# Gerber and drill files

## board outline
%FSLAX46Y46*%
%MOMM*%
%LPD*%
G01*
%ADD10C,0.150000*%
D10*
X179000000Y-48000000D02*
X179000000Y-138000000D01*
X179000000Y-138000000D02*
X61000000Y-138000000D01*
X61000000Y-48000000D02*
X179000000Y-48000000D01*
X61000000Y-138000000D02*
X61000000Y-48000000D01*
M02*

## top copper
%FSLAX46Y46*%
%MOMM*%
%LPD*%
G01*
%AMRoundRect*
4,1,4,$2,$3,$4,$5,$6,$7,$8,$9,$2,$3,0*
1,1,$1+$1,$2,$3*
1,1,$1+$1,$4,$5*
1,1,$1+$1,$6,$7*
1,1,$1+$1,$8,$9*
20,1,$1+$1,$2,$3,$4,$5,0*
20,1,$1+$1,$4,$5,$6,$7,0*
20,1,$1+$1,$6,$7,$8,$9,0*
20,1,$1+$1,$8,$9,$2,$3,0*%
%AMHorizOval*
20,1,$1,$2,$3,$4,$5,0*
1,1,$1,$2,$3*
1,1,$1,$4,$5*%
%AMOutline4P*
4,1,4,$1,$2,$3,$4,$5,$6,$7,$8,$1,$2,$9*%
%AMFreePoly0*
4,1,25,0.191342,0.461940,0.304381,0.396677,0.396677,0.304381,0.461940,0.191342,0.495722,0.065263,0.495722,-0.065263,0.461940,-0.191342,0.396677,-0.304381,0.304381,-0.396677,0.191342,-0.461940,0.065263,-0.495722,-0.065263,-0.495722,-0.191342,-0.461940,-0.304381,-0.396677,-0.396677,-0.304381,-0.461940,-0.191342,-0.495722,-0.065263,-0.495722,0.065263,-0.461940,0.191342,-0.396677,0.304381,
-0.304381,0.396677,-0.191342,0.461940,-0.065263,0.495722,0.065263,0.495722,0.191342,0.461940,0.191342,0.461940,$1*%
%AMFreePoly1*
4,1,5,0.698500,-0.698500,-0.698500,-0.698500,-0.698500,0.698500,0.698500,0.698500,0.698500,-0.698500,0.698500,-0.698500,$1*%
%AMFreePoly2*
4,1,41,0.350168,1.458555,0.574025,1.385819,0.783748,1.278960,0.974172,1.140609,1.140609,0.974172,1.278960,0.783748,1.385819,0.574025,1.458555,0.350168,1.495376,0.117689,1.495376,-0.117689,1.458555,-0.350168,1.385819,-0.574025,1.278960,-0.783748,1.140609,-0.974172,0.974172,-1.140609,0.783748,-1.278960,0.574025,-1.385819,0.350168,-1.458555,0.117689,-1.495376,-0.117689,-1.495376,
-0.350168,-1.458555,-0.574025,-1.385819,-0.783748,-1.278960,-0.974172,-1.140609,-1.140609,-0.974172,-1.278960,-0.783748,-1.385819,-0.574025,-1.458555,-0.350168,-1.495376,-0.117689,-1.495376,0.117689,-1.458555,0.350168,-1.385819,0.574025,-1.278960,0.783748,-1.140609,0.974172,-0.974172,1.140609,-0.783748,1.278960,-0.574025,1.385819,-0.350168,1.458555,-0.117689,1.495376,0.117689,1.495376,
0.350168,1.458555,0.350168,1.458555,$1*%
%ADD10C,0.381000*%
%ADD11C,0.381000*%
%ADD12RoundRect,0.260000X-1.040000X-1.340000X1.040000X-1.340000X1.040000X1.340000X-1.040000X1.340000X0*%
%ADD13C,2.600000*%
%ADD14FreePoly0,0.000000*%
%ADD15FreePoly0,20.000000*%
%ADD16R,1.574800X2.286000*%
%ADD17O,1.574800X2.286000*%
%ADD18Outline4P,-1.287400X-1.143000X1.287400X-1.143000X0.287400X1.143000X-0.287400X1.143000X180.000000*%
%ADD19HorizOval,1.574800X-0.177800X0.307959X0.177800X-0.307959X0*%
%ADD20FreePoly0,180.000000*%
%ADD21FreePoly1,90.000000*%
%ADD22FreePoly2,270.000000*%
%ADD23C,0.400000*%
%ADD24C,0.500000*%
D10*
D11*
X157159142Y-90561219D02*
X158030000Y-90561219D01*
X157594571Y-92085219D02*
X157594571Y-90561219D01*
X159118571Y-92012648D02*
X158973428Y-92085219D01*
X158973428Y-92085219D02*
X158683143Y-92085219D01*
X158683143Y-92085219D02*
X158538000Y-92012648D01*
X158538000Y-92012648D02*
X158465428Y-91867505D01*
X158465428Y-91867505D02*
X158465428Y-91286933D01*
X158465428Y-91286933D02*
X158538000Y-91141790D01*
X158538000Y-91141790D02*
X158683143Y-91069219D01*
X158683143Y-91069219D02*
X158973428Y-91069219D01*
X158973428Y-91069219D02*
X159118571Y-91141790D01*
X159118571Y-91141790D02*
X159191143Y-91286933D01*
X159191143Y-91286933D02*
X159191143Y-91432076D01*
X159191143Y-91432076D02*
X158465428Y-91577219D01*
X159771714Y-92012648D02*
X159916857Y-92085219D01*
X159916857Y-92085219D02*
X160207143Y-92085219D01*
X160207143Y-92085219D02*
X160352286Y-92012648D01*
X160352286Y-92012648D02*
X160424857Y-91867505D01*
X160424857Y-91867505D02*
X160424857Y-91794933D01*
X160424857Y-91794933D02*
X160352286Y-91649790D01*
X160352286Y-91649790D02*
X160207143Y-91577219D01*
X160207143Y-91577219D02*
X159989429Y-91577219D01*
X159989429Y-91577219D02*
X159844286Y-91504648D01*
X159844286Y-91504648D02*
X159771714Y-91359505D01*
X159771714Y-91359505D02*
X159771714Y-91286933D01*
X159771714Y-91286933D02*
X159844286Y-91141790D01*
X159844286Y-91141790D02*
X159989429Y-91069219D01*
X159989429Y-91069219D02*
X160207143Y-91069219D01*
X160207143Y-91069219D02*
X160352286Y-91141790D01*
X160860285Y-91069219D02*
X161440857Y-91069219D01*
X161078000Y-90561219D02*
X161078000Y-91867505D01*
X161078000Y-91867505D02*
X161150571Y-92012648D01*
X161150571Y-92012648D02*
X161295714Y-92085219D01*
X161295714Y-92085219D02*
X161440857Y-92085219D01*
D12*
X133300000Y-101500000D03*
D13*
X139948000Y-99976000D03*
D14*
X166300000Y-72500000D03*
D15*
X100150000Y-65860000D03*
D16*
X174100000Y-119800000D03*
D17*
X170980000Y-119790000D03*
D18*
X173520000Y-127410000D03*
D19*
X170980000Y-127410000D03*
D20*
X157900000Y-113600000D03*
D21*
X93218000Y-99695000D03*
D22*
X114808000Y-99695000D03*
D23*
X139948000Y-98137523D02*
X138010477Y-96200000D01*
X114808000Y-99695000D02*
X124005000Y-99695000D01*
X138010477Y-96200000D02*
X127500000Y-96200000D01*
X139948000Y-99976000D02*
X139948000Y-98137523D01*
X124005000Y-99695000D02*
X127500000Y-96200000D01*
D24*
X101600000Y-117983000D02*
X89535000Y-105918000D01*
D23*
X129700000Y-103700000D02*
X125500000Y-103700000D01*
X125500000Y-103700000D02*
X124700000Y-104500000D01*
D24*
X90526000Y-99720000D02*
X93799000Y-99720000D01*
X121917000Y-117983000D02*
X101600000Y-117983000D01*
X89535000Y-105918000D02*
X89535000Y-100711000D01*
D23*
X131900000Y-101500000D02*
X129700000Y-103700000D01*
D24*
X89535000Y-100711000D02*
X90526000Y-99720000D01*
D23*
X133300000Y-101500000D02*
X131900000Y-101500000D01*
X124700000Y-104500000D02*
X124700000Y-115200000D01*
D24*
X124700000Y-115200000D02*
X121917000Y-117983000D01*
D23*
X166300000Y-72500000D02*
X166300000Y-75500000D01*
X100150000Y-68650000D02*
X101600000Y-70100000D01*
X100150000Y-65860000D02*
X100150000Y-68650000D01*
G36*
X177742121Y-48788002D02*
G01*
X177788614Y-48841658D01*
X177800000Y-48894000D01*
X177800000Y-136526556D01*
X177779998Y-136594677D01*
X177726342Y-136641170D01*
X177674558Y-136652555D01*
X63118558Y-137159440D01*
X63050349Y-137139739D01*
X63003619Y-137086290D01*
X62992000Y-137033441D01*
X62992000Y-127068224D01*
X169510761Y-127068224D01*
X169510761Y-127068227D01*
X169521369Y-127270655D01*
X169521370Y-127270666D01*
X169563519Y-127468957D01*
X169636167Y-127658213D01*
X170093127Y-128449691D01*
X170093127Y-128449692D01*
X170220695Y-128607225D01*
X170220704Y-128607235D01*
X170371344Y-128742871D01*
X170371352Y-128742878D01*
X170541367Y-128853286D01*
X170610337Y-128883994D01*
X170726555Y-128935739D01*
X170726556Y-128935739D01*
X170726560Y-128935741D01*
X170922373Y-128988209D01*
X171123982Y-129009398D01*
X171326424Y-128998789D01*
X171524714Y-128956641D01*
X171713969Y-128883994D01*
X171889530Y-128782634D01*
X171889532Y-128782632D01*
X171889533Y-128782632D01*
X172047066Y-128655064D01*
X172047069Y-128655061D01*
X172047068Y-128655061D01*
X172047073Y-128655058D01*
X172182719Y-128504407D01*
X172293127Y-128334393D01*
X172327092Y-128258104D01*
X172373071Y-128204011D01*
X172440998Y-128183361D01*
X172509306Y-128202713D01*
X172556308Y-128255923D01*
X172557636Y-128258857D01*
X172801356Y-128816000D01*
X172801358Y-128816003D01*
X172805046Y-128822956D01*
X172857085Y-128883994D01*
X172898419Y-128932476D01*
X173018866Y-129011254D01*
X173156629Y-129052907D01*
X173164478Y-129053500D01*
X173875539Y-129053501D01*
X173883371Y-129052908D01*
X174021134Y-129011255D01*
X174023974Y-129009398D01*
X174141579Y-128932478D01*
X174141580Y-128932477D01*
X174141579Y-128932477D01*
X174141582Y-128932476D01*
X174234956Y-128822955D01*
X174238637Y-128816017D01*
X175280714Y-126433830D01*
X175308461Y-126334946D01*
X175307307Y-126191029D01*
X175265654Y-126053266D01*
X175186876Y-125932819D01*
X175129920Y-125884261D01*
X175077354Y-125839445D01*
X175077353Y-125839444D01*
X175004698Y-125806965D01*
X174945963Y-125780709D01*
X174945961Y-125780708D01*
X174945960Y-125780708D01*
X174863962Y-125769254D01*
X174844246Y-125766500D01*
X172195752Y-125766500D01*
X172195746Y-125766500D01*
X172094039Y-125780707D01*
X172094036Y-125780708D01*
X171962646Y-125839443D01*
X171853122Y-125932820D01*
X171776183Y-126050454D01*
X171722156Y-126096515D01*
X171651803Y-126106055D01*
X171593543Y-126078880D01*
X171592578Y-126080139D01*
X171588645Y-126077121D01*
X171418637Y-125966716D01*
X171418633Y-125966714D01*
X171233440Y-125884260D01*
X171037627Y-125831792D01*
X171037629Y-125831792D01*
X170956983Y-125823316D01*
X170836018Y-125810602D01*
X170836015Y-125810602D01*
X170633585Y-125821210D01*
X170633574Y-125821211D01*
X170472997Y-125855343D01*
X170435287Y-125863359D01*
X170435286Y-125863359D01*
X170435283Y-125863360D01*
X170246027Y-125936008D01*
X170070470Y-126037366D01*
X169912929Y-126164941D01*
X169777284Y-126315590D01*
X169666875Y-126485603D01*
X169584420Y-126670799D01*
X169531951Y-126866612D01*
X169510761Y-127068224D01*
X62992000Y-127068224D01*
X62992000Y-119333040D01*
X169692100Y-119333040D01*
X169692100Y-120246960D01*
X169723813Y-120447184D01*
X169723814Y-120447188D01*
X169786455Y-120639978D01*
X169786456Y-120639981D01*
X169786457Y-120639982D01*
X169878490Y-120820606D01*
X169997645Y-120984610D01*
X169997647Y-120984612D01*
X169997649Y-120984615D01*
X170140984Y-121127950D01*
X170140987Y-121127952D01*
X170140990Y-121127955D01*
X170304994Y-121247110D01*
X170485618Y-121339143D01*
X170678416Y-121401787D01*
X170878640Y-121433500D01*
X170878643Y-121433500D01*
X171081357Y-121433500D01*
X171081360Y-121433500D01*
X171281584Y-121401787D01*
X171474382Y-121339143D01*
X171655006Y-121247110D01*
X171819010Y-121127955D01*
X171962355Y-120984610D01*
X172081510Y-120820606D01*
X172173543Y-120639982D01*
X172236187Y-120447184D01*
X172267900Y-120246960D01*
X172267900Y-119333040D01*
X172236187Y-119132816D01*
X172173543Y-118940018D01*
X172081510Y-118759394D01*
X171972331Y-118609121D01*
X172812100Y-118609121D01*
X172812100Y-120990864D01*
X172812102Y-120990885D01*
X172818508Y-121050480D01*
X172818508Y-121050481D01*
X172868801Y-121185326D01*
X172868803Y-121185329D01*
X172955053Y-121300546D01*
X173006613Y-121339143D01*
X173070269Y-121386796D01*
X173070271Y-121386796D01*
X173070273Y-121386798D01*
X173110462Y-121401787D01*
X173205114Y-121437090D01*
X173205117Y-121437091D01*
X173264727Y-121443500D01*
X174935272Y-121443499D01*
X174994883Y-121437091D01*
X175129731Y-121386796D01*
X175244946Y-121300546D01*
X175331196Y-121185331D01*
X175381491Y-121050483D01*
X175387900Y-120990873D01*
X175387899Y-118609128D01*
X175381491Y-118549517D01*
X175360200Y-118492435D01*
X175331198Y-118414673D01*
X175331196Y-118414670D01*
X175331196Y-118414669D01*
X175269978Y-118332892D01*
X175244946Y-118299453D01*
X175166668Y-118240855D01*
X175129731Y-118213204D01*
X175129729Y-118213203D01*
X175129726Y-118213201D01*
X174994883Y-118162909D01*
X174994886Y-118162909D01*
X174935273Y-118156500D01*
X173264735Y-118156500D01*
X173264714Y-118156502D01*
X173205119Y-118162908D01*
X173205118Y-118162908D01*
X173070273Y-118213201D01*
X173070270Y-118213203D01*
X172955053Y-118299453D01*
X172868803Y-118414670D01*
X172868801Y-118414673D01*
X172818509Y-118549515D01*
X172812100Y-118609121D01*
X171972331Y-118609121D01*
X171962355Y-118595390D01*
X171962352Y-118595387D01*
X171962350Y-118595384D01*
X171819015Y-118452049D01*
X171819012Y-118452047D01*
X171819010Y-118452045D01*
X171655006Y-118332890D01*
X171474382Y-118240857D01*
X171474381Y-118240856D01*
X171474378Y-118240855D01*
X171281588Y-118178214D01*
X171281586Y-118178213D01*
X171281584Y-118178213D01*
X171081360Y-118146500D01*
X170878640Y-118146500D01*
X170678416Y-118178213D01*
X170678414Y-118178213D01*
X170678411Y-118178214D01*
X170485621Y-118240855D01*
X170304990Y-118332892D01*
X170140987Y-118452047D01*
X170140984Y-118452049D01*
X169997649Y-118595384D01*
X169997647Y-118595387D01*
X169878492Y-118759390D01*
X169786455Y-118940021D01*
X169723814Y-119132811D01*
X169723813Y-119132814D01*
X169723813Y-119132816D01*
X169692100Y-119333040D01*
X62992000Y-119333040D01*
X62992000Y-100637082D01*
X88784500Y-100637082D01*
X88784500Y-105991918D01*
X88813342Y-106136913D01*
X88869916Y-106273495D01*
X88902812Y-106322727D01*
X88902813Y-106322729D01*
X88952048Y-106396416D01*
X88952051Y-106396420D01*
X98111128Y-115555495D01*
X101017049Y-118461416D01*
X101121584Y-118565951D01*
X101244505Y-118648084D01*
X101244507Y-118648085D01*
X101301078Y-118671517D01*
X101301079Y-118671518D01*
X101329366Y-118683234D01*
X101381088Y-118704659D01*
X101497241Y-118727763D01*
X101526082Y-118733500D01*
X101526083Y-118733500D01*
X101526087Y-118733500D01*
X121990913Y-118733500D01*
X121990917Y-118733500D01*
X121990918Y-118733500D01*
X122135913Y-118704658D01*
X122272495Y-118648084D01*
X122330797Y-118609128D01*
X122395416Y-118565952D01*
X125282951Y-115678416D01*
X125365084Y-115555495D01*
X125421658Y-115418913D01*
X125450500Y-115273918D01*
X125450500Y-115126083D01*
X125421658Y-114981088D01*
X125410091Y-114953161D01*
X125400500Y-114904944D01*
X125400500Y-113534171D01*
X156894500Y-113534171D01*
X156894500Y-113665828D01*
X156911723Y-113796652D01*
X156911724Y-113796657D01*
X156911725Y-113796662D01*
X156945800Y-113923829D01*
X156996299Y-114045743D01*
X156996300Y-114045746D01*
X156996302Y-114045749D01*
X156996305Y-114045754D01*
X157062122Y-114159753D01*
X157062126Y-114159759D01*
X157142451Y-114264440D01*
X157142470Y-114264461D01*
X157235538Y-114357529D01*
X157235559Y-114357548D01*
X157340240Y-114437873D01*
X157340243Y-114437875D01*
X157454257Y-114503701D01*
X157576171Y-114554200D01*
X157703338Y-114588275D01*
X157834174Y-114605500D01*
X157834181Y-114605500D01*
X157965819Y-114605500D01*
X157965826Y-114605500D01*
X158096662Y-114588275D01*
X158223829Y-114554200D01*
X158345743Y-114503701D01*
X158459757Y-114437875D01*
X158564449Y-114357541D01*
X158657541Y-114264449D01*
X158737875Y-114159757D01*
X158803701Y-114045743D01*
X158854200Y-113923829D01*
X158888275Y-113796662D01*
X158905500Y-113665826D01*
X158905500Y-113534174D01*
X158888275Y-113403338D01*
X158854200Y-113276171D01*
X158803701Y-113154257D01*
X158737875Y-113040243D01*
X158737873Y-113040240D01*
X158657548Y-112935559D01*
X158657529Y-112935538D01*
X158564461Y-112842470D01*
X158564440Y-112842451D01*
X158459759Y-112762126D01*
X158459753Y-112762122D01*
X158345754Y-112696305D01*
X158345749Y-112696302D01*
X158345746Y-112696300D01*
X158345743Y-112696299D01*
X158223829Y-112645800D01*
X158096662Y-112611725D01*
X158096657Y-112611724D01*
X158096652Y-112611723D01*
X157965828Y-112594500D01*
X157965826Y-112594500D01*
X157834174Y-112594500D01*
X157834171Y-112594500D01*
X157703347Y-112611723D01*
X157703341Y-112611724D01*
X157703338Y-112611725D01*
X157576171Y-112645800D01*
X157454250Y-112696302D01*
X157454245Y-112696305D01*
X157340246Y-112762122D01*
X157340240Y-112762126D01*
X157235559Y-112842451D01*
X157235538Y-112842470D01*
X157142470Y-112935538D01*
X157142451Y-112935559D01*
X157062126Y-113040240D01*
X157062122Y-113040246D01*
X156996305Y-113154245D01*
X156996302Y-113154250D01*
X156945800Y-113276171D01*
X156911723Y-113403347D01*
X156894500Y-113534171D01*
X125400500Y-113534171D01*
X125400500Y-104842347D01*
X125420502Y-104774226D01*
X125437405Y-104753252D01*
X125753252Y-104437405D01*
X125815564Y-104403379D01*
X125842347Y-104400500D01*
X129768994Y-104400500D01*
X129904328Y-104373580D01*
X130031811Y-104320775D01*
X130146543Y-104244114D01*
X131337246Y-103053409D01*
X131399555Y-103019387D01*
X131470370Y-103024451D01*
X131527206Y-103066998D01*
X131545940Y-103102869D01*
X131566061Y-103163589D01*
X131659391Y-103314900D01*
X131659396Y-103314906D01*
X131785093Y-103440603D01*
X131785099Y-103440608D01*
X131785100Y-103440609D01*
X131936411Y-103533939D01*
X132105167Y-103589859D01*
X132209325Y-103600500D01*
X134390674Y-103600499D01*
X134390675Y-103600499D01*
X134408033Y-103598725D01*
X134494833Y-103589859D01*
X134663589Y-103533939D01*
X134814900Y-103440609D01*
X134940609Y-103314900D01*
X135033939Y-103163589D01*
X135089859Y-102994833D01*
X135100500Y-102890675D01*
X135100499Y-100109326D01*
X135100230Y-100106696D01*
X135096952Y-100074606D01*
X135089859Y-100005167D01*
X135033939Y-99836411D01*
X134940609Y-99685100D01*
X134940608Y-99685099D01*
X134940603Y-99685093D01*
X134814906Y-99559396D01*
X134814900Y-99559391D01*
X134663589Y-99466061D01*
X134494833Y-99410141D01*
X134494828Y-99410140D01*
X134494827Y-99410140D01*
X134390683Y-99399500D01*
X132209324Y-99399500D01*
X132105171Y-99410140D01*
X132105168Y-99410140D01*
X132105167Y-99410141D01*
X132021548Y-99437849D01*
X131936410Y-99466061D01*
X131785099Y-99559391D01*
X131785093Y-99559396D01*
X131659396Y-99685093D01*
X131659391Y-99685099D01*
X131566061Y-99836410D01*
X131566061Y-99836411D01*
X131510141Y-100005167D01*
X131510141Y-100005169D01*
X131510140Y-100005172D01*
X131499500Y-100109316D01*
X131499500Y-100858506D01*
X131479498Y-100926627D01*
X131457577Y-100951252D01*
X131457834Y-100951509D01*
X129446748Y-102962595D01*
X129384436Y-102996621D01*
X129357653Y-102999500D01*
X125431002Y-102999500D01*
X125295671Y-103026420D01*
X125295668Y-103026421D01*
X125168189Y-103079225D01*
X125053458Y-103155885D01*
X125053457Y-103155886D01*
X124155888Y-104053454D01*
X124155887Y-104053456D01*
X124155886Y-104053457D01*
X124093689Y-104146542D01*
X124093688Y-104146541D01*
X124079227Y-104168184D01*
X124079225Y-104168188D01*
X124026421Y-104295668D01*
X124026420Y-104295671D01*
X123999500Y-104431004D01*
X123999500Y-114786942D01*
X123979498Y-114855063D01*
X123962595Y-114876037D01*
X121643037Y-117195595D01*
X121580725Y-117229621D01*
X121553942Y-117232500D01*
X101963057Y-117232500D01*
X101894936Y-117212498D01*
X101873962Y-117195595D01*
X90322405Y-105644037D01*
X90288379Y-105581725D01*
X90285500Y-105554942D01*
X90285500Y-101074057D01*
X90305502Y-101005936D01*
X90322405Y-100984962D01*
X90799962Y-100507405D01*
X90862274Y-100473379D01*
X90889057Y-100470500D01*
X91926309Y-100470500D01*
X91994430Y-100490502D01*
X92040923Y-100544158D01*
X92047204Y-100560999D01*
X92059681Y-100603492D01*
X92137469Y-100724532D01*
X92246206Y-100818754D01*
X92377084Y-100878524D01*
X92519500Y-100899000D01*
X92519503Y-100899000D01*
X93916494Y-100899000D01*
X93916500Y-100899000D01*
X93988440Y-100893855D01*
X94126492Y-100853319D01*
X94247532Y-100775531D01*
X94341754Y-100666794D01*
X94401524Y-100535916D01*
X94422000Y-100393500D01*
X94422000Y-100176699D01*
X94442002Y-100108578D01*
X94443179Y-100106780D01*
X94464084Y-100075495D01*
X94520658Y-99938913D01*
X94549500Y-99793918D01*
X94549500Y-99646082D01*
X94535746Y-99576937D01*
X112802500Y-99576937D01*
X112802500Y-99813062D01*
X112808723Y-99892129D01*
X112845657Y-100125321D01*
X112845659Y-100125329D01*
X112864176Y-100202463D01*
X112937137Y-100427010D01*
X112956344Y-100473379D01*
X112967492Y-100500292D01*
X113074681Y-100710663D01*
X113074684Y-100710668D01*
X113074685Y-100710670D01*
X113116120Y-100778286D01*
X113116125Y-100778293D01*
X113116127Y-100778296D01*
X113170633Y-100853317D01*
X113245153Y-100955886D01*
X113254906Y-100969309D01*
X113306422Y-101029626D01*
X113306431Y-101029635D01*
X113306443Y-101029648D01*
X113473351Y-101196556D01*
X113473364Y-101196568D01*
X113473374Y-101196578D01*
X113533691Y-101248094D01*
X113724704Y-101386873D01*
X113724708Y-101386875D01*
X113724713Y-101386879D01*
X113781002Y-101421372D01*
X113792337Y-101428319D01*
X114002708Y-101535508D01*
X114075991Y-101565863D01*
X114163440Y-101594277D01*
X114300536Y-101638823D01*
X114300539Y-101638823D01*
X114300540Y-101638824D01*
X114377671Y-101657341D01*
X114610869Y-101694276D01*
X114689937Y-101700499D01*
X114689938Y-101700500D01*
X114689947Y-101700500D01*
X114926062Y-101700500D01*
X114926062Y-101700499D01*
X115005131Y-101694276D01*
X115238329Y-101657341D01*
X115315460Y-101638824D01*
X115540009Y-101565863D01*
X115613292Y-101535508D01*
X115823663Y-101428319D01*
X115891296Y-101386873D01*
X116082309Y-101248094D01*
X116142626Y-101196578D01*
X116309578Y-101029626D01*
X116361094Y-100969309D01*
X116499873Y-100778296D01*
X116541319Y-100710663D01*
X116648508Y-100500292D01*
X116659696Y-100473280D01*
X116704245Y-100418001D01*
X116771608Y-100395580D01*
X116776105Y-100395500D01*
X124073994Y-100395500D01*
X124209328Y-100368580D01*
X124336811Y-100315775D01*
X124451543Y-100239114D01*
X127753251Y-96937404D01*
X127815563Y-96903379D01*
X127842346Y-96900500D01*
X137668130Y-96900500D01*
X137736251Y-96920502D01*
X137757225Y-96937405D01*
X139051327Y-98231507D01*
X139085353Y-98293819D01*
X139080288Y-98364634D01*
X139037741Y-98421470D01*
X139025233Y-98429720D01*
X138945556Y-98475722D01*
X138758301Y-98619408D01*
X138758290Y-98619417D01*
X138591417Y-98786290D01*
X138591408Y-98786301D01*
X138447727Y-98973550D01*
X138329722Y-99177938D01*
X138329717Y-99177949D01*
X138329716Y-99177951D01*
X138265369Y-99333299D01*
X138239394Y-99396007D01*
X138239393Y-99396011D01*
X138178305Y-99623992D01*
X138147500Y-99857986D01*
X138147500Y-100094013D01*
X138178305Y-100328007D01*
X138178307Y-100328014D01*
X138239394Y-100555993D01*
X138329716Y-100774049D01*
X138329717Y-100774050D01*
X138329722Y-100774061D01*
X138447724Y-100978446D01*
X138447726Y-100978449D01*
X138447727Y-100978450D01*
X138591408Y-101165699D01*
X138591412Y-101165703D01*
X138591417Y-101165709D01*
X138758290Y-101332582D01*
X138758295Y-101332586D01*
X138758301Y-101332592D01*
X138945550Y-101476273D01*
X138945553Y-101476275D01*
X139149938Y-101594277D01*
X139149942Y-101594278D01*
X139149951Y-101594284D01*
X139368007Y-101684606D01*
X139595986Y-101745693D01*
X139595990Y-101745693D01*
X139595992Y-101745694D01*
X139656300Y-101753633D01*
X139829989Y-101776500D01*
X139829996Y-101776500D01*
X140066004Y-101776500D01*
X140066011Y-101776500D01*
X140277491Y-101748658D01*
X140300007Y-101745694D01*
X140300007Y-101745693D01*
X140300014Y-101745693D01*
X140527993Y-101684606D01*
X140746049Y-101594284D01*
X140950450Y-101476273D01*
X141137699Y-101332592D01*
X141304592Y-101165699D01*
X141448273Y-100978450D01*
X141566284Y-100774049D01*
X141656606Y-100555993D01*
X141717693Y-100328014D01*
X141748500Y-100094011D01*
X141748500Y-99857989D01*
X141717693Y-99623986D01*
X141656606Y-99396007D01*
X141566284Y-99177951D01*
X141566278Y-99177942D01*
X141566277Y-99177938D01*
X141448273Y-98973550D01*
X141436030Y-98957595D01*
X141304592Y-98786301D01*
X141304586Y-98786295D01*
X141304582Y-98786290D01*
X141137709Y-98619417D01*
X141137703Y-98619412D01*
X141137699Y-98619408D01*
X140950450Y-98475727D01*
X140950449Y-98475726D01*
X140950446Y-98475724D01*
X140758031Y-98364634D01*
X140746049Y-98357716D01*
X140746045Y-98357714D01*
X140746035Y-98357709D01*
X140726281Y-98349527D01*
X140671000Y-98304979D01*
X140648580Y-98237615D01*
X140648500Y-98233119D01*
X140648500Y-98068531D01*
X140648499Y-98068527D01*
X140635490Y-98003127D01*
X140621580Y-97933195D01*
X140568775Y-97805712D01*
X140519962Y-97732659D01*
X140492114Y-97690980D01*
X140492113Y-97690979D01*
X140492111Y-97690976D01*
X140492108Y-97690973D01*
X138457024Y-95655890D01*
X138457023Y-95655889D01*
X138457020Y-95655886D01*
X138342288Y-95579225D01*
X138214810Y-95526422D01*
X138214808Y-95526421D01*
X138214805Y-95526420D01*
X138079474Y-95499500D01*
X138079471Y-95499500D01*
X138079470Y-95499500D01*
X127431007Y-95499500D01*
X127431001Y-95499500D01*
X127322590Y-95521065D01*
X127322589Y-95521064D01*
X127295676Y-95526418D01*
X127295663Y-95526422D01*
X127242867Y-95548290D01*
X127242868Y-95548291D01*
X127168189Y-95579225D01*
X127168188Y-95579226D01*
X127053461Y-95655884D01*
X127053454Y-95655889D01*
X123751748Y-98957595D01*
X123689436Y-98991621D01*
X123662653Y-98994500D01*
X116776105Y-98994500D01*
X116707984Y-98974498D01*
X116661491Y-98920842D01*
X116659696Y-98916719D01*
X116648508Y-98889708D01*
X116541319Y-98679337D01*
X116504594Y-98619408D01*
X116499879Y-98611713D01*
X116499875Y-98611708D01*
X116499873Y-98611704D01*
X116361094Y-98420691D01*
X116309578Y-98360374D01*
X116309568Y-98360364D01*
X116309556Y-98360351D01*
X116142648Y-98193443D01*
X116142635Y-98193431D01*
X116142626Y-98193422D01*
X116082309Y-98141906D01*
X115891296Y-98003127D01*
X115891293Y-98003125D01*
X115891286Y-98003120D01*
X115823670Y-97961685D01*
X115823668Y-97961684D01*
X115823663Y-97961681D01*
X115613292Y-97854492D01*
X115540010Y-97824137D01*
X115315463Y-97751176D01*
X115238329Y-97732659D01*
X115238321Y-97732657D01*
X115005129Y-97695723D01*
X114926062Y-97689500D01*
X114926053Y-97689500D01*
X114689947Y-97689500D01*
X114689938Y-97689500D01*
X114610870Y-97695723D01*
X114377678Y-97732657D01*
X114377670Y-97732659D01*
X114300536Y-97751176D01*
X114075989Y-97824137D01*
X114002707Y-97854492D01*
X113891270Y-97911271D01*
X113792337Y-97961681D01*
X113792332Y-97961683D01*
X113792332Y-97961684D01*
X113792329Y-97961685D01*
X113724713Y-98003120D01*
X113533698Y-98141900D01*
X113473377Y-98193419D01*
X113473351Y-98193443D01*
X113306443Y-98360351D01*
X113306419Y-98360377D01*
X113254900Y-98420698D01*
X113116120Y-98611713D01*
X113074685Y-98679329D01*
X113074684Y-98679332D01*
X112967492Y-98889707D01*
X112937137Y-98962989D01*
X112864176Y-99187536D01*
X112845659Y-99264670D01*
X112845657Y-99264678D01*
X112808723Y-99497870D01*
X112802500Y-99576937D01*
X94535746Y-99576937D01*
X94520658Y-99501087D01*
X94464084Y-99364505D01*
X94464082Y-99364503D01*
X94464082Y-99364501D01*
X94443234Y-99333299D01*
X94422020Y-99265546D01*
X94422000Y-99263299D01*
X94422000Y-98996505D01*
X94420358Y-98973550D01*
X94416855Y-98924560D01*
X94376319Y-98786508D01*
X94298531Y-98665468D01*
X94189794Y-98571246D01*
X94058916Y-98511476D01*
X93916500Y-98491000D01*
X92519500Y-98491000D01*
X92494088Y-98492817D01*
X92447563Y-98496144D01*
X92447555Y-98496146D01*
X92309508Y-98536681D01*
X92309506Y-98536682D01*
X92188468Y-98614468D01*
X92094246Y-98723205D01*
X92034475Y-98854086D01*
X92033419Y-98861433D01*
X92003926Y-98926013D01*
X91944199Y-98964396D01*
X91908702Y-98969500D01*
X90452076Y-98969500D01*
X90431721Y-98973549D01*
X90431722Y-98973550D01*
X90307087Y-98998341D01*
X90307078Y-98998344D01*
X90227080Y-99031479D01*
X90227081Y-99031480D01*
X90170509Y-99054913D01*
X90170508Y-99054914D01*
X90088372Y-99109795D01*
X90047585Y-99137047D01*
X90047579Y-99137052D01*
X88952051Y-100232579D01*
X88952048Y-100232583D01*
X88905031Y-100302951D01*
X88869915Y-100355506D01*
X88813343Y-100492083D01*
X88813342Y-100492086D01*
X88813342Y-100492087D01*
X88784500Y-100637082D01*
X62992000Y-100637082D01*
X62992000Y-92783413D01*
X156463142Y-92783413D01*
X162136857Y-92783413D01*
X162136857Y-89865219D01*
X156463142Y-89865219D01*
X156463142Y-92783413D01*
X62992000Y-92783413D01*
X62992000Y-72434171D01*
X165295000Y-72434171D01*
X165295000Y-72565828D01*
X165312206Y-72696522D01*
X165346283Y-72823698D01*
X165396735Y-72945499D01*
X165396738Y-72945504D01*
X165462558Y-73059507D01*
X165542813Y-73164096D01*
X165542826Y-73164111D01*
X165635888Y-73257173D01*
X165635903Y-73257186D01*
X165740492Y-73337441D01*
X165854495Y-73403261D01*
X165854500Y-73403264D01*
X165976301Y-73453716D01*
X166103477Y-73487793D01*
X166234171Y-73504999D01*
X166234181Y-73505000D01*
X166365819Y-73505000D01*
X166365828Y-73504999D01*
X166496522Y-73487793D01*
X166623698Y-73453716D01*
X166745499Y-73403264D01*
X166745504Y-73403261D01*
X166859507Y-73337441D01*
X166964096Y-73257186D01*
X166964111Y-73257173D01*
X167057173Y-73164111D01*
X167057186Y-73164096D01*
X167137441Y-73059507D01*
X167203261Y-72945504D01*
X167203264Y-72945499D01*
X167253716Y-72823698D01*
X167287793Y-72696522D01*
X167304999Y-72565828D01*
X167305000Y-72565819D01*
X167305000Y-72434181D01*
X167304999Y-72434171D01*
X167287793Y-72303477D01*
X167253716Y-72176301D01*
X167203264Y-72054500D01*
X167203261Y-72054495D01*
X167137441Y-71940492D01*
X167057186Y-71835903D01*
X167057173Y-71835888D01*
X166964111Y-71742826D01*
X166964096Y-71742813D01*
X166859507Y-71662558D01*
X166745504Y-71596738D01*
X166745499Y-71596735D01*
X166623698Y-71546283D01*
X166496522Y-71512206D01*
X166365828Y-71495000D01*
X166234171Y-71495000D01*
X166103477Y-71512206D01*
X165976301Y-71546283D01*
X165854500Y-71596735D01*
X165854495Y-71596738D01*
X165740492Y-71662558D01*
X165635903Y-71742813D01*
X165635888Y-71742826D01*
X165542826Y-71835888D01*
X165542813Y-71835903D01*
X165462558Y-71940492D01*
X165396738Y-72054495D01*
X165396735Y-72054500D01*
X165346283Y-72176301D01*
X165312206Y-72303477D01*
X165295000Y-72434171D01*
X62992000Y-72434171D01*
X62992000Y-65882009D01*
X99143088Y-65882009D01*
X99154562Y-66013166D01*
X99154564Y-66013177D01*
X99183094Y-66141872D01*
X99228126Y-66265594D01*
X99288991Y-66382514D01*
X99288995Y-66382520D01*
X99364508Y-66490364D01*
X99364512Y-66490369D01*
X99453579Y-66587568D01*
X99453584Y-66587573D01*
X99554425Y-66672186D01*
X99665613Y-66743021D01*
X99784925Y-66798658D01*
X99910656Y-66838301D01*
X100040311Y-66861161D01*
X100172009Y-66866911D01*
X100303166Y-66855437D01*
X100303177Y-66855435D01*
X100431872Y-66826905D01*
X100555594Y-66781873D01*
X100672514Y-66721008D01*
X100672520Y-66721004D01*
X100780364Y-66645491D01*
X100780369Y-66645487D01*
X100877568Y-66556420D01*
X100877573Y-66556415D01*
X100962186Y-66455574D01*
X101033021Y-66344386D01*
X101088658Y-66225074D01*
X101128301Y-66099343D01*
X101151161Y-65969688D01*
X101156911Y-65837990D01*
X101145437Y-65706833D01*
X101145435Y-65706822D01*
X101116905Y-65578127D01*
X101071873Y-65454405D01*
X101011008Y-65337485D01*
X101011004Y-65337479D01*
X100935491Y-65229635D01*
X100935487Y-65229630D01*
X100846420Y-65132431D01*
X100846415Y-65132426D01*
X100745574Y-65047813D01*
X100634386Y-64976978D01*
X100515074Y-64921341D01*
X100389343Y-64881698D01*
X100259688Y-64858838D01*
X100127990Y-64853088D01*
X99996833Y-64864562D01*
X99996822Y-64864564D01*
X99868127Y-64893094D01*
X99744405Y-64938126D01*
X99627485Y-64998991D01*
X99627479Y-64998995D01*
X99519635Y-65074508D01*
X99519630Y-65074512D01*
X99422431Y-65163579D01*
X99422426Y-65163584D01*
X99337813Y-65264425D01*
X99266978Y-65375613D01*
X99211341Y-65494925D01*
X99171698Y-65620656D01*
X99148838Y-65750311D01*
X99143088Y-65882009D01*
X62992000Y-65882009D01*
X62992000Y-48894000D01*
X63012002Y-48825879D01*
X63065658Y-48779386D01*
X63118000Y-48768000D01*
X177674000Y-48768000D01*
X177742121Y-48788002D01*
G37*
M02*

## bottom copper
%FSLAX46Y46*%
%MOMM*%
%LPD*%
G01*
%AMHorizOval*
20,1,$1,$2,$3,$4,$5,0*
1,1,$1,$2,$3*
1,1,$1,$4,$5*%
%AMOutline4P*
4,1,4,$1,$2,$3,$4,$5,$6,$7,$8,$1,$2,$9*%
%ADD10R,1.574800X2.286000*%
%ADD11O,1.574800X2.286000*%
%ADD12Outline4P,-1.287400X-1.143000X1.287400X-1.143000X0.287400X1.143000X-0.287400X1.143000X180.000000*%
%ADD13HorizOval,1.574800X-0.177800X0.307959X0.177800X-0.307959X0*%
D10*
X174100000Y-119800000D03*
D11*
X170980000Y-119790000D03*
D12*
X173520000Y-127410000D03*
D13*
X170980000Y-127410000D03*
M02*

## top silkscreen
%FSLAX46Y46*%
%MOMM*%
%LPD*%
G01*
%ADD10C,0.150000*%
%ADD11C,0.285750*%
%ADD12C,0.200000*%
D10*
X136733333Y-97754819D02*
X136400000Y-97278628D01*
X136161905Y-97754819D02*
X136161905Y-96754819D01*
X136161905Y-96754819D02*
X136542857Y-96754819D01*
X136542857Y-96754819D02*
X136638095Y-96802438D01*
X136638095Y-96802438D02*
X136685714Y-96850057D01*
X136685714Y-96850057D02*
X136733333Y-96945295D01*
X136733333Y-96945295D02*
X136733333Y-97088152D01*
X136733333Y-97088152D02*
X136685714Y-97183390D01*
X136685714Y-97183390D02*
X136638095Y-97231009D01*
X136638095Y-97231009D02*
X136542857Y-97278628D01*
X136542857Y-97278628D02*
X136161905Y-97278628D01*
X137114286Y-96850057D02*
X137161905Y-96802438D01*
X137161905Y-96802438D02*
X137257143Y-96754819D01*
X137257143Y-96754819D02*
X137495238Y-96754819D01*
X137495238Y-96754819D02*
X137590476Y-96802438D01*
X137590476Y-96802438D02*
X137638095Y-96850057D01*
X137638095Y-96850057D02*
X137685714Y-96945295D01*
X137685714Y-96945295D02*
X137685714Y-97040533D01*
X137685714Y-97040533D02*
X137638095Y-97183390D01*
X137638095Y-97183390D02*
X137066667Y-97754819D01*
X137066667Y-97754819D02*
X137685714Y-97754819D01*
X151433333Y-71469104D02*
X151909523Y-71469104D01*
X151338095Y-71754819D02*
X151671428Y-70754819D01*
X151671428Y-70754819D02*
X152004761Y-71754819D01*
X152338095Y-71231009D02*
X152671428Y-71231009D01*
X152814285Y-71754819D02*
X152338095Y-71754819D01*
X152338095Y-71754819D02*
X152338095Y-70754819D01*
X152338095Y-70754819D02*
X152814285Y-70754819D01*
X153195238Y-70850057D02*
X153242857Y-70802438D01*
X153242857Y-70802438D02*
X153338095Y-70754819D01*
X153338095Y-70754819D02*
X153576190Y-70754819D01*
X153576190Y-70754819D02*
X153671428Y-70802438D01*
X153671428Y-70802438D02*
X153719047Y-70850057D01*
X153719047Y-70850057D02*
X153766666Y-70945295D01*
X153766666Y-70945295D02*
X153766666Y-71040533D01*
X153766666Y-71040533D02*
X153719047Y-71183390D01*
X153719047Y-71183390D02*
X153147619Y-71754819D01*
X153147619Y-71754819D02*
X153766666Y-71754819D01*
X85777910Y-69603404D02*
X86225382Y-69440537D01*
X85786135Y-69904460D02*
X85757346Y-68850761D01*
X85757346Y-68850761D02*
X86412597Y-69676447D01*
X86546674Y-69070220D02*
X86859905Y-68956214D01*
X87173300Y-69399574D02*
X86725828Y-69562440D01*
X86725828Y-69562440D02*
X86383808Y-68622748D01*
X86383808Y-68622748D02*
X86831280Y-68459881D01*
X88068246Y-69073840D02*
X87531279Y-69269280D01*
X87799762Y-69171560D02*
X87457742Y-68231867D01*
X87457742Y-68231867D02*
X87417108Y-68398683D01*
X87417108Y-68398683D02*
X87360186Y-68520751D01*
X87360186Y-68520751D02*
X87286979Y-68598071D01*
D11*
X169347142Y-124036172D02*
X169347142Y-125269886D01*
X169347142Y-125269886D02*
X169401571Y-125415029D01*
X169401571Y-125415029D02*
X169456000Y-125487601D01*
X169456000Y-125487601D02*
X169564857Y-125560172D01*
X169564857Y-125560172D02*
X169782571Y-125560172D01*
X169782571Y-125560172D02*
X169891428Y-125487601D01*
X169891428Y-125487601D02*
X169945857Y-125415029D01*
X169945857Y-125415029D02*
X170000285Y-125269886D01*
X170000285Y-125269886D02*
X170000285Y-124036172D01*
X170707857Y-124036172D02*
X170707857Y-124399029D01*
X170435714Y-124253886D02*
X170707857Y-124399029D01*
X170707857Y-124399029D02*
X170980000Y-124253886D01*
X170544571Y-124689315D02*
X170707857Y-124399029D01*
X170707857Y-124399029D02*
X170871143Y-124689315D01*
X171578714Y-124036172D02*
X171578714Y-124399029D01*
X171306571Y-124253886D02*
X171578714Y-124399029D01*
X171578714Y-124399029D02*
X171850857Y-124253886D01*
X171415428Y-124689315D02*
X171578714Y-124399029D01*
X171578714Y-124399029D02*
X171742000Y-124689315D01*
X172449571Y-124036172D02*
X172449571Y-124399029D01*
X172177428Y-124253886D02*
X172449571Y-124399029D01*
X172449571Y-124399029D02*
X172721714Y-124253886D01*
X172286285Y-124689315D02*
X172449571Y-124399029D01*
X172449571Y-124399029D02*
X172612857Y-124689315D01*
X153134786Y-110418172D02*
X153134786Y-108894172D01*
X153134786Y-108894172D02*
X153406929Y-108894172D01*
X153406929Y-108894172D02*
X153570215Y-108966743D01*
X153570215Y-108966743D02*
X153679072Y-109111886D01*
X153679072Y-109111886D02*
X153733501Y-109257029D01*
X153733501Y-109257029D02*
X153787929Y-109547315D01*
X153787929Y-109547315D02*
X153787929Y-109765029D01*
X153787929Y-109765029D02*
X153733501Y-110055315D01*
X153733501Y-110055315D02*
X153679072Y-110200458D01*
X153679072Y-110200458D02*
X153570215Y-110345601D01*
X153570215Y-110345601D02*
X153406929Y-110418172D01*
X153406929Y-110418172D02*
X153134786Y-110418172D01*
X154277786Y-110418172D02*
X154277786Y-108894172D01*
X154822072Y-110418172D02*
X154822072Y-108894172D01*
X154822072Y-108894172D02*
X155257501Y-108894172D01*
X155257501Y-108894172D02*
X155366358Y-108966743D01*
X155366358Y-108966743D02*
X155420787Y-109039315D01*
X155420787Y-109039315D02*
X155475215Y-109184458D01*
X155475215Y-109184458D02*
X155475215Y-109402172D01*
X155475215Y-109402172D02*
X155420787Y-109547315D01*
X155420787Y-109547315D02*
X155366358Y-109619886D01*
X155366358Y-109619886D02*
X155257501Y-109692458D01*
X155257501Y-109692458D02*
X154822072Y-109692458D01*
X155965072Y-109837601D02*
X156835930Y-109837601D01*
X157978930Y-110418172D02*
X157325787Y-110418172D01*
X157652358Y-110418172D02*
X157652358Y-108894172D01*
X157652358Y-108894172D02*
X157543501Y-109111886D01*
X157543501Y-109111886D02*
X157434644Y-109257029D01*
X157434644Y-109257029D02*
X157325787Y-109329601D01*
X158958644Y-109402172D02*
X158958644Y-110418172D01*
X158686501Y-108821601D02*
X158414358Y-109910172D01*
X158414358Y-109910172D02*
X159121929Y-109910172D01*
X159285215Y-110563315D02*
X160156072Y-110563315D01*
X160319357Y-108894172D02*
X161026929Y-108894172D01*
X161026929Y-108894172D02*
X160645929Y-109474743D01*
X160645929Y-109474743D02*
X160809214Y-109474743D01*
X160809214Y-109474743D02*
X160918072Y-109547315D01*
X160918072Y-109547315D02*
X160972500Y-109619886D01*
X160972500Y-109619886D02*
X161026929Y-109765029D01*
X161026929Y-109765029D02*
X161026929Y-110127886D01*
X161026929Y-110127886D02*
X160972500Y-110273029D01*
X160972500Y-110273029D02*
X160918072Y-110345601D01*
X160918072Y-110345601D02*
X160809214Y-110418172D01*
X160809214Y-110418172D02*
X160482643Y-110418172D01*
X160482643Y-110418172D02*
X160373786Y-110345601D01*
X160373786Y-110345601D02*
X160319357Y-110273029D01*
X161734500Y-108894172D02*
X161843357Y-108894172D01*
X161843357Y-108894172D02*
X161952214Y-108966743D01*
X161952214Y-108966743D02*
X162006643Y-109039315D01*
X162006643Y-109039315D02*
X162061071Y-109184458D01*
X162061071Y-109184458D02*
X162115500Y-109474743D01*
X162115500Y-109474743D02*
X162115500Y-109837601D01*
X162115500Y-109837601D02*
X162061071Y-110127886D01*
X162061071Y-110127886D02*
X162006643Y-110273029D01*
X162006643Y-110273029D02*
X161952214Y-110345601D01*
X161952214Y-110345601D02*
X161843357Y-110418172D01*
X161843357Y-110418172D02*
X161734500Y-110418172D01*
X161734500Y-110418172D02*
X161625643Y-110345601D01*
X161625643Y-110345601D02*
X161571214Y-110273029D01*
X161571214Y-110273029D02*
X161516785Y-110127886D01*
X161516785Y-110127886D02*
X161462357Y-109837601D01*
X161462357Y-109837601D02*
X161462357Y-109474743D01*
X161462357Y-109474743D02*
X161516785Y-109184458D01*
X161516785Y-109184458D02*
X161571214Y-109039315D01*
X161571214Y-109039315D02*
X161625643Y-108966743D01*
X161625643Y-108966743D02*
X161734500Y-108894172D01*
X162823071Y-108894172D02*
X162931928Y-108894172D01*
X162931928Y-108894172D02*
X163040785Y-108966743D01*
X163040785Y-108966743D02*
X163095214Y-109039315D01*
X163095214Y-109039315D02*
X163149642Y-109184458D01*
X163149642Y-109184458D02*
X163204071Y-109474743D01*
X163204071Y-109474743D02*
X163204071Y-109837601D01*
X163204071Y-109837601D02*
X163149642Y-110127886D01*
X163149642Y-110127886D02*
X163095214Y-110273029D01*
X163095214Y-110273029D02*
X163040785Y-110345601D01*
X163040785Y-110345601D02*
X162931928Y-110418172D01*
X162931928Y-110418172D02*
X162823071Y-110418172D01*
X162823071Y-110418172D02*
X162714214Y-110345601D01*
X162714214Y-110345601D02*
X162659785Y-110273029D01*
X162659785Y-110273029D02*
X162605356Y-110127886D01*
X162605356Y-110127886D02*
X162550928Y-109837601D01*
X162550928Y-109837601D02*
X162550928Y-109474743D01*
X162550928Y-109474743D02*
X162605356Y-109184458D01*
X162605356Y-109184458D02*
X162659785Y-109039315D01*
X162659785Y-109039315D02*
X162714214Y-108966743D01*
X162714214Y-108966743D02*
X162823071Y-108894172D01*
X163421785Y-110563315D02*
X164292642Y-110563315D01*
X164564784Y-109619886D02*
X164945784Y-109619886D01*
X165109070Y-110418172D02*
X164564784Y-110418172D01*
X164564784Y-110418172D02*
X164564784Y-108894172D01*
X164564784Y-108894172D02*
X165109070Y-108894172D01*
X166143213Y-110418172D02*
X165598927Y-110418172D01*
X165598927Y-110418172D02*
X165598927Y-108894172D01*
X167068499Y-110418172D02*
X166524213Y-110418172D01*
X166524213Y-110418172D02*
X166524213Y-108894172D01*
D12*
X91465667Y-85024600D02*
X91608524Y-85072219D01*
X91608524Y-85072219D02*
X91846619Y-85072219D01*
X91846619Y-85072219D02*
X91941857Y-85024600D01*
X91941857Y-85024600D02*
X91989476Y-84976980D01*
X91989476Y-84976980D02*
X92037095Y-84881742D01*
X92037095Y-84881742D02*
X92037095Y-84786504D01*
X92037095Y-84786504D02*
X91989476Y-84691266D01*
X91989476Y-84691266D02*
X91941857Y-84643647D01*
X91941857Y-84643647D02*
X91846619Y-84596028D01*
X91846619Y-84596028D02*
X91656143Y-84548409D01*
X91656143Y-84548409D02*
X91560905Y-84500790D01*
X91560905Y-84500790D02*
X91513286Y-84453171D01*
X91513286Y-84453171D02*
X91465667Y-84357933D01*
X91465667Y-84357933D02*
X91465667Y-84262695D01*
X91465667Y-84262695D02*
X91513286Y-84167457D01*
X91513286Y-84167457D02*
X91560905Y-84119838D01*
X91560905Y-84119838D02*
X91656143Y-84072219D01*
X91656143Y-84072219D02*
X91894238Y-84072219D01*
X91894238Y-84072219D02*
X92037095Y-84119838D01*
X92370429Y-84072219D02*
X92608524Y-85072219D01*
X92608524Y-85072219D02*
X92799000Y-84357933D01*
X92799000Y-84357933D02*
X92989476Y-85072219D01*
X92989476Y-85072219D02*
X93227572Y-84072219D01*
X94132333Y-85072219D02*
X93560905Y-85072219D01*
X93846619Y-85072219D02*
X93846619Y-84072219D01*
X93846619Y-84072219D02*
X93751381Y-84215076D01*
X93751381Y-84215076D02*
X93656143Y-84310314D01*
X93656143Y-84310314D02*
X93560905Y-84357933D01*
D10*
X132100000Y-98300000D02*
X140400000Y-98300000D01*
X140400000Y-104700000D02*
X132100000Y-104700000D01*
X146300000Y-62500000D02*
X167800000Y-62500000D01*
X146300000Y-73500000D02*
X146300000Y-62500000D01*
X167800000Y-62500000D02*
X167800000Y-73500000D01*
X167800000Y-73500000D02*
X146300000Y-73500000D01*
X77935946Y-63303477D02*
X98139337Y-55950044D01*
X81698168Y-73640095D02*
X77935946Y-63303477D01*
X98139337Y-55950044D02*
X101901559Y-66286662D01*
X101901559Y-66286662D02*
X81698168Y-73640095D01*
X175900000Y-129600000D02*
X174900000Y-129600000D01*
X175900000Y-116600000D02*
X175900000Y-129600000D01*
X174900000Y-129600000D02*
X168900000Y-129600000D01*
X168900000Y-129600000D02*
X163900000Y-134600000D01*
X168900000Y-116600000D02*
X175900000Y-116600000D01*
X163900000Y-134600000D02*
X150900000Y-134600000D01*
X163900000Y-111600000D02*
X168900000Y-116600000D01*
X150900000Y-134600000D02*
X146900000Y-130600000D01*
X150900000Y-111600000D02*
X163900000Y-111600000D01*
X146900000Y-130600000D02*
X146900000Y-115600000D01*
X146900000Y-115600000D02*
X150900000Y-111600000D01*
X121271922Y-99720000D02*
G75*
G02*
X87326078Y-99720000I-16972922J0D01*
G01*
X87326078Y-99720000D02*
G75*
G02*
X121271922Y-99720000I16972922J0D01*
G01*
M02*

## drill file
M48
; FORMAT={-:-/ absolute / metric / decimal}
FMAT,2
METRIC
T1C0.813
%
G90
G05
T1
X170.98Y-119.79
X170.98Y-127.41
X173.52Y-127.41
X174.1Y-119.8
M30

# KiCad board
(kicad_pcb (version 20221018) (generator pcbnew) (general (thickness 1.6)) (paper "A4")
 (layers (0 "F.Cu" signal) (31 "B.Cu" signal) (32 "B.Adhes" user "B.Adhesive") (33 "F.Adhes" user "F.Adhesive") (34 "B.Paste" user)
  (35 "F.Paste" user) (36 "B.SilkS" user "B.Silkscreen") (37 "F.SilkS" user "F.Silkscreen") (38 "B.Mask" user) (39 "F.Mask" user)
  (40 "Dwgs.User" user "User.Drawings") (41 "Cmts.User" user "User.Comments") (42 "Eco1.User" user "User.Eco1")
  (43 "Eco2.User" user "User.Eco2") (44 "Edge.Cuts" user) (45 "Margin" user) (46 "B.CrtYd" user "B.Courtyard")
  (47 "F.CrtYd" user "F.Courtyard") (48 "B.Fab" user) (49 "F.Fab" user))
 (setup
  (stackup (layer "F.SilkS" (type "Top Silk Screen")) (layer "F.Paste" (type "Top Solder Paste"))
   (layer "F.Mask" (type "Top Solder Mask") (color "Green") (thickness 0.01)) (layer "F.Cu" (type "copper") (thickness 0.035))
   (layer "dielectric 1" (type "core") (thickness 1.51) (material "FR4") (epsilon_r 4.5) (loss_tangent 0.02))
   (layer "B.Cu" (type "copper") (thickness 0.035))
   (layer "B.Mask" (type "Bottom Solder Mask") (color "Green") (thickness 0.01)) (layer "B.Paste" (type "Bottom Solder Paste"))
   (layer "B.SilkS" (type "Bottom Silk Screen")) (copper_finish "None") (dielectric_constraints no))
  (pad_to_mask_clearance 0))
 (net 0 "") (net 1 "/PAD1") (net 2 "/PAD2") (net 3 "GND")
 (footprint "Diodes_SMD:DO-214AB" (layer "F.Cu") (at 136.9 101.5)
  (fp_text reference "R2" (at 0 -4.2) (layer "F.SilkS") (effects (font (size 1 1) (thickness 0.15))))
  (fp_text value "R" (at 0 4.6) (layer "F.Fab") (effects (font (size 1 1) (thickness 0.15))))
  (fp_line (start -4.8 -3.2) (end 3.5 -3.2) (stroke (width 0.15) (type solid)) (layer "F.SilkS"))
  (fp_line (start 3.5 3.2) (end -4.8 3.2) (stroke (width 0.15) (type solid)) (layer "F.SilkS"))
  (pad "1" smd roundrect (at -3.6 0) (size 2.6 3.2) (layers "F.Cu" "F.Paste" "F.Mask") (roundrect_rratio 0.1) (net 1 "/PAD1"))
  (pad "2" smd circle (at 3.048 -1.524) (size 2.6 2.6) (layers "F.Cu" "F.Paste" "F.Mask") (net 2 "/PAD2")))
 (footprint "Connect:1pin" (layer "F.Cu") (at 166.3 72.5)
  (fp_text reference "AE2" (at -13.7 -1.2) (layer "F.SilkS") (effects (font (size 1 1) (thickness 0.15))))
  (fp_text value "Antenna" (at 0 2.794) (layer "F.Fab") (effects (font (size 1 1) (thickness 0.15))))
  (fp_line (start -20 -10) (end 1.5 -10) (stroke (width 0.15) (type solid)) (layer "F.SilkS"))
  (fp_line (start -20 1) (end -20 -10) (stroke (width 0.15) (type solid)) (layer "F.SilkS"))
  (fp_line (start 1.5 -10) (end 1.5 1) (stroke (width 0.15) (type solid)) (layer "F.SilkS"))
  (fp_line (start 1.5 1) (end -20 1) (stroke (width 0.15) (type solid)) (layer "F.SilkS"))
  (pad "1" smd custom (at 0 0) (size 1 1) (layers "F.Cu" "F.Paste" "F.Mask") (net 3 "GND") (zone_connect 0) (thermal_bridge_angle 45)
   (options (clearance outline) (anchor circle)) (primitives)))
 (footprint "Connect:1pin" (layer "F.Cu") (at 100.15 65.86 20)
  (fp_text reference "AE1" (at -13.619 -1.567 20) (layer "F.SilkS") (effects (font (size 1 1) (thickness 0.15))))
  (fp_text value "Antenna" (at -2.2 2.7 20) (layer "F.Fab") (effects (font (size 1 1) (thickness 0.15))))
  (fp_line (start -20 -10) (end 1.5 -10) (stroke (width 0.15) (type solid)) (layer "F.SilkS"))
  (fp_line (start -20 1) (end -20 -10) (stroke (width 0.15) (type solid)) (layer "F.SilkS"))
  (fp_line (start 1.5 -10) (end 1.5 1) (stroke (width 0.15) (type solid)) (layer "F.SilkS"))
  (fp_line (start 1.5 1) (end -20 1) (stroke (width 0.15) (type solid)) (layer "F.SilkS"))
  (pad "1" connect custom (at 0 0 20) (size 1 1) (layers "F.Cu" "F.Mask") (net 3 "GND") (zone_connect 0) (thermal_bridge_angle 45)
   (options (clearance outline) (anchor circle)) (primitives)))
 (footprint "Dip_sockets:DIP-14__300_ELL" (layer "F.Cu") (at 165.9 123.6 180)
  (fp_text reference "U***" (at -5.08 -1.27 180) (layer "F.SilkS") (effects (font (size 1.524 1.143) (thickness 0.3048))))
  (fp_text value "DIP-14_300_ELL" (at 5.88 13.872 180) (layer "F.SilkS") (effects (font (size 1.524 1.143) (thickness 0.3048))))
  (fp_line (start -10 -6) (end -9 -6) (stroke (width 0.15) (type solid)) (layer "F.SilkS"))
  (fp_line (start -10 7) (end -10 -6) (stroke (width 0.15) (type solid)) (layer "F.SilkS"))
  (fp_line (start -9 -6) (end -3 -6) (stroke (width 0.15) (type solid)) (layer "F.SilkS"))
  (fp_line (start -3 -6) (end 2 -11) (stroke (width 0.15) (type solid)) (layer "F.SilkS"))
  (fp_line (start -3 7) (end -10 7) (stroke (width 0.15) (type solid)) (layer "F.SilkS"))
  (fp_line (start 2 -11) (end 15 -11) (stroke (width 0.15) (type solid)) (layer "F.SilkS"))
  (fp_line (start 2 12) (end -3 7) (stroke (width 0.15) (type solid)) (layer "F.SilkS"))
  (fp_line (start 15 -11) (end 19 -7) (stroke (width 0.15) (type solid)) (layer "F.SilkS"))
  (fp_line (start 15 12) (end 2 12) (stroke (width 0.15) (type solid)) (layer "F.SilkS"))
  (fp_line (start 19 -7) (end 19 8) (stroke (width 0.15) (type solid)) (layer "F.SilkS"))
  (fp_line (start 19 8) (end 15 12) (stroke (width 0.15) (type solid)) (layer "F.SilkS"))
  (pad "1" thru_hole rect (at -8.2 3.8 180) (size 1.5748 2.286) (drill 0.8128) (layers "*.Cu" "*.Mask"))
  (pad "2" thru_hole oval (at -5.08 3.81 180) (size 1.5748 2.286) (drill 0.8128) (layers "*.Cu" "*.Mask"))
  (pad "3" thru_hole trapezoid (at -7.62 -3.81 180) (size 1.5748 2.286) (rect_delta 0 1) (drill 0.8128) (layers "*.Cu" "*.Mask"))
  (pad "4" thru_hole oval (at -5.08 -3.81 210) (size 1.5748 2.286) (drill 0.8128) (layers "*.Cu" "*.Mask"))
  (pad "5" connect custom (at 8 10 180) (size 1 1) (layers "F.Cu" "F.Mask") (zone_connect 0) (thermal_bridge_angle 45)
   (options (clearance convexhull) (anchor circle)) (primitives)))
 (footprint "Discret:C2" (layer "F.Cu") (at 104.299 99.72)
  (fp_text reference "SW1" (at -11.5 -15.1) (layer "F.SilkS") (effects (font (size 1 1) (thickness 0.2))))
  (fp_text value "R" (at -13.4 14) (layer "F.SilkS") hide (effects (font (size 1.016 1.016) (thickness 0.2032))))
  (fp_circle (center 0 0) (end 12.065 -11.938) (stroke (width 0.15) (type solid)) (fill none) (layer "F.SilkS"))
  (pad "1" connect custom (at -11.081 -0.025 90) (size 1.397 1.397) (layers "F.Cu" "F.Mask") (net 1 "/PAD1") (solder_mask_margin 0.5)
   (zone_connect 0) (thermal_bridge_angle 45) (options (clearance convexhull) (anchor rect)) (primitives))
  (pad "2" connect custom (at 10.509 -0.025 270) (size 3 3) (layers "F.Cu" "F.Mask") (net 2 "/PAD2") (zone_connect 0)
   (thermal_bridge_angle 45) (options (clearance outline) (anchor circle)) (primitives)))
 (gr_line (start 179 48) (end 179 138) (stroke (width 0.15) (type solid)) (layer "Edge.Cuts"))
 (gr_line (start 179 138) (end 61 138) (stroke (width 0.15) (type solid)) (layer "Edge.Cuts"))
 (gr_line (start 61 48) (end 179 48) (stroke (width 0.15) (type solid)) (layer "Edge.Cuts"))
 (gr_line (start 61 138) (end 61 48) (stroke (width 0.15) (type solid)) (layer "Edge.Cuts"))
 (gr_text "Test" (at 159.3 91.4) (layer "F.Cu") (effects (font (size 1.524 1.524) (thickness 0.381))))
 (segment (start 139.948 98.137523) (end 138.010477 96.2) (width 0.4) (layer "F.Cu") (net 2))
 (segment (start 114.808 99.695) (end 124.005 99.695) (width 0.4) (layer "F.Cu") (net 2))
 (segment (start 138.010477 96.2) (end 127.5 96.2) (width 0.4) (layer "F.Cu") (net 2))
 (segment (start 139.948 99.976) (end 139.948 98.137523) (width 0.4) (layer "F.Cu") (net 2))
 (segment (start 124.005 99.695) (end 127.5 96.2) (width 0.4) (layer "F.Cu") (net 2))
 (segment (start 101.6 117.983) (end 89.535 105.918) (width 0.5) (layer "F.Cu") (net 1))
 (segment (start 129.7 103.7) (end 125.5 103.7) (width 0.4) (layer "F.Cu") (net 1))
 (segment (start 125.5 103.7) (end 124.7 104.5) (width 0.4) (layer "F.Cu") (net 1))
 (segment (start 90.526 99.72) (end 93.799 99.72) (width 0.5) (layer "F.Cu") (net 1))
 (segment (start 121.917 117.983) (end 101.6 117.983) (width 0.5) (layer "F.Cu") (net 1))
 (segment (start 89.535 105.918) (end 89.535 100.711) (width 0.5) (layer "F.Cu") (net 1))
 (segment (start 131.9 101.5) (end 129.7 103.7) (width 0.4) (layer "F.Cu") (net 1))
 (segment (start 89.535 100.711) (end 90.526 99.72) (width 0.5) (layer "F.Cu") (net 1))
 (segment (start 133.3 101.5) (end 131.9 101.5) (width 0.4) (layer "F.Cu") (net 1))
 (segment (start 124.7 104.5) (end 124.7 115.2) (width 0.4) (layer "F.Cu") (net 1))
 (segment (start 124.7 115.2) (end 121.917 117.983) (width 0.5) (layer "F.Cu") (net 1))
 (segment (start 166.3 72.5) (end 166.3 75.5) (width 0.4) (layer "F.Cu") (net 3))
 (segment (start 100.15 68.65) (end 101.6 70.1) (width 0.4) (layer "F.Cu") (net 3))
 (segment (start 100.15 65.86) (end 100.15 68.65) (width 0.4) (layer "F.Cu") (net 3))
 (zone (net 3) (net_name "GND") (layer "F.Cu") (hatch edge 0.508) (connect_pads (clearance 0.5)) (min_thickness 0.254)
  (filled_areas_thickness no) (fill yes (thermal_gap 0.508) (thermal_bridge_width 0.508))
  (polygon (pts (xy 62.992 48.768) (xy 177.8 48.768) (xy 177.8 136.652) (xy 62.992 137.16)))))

